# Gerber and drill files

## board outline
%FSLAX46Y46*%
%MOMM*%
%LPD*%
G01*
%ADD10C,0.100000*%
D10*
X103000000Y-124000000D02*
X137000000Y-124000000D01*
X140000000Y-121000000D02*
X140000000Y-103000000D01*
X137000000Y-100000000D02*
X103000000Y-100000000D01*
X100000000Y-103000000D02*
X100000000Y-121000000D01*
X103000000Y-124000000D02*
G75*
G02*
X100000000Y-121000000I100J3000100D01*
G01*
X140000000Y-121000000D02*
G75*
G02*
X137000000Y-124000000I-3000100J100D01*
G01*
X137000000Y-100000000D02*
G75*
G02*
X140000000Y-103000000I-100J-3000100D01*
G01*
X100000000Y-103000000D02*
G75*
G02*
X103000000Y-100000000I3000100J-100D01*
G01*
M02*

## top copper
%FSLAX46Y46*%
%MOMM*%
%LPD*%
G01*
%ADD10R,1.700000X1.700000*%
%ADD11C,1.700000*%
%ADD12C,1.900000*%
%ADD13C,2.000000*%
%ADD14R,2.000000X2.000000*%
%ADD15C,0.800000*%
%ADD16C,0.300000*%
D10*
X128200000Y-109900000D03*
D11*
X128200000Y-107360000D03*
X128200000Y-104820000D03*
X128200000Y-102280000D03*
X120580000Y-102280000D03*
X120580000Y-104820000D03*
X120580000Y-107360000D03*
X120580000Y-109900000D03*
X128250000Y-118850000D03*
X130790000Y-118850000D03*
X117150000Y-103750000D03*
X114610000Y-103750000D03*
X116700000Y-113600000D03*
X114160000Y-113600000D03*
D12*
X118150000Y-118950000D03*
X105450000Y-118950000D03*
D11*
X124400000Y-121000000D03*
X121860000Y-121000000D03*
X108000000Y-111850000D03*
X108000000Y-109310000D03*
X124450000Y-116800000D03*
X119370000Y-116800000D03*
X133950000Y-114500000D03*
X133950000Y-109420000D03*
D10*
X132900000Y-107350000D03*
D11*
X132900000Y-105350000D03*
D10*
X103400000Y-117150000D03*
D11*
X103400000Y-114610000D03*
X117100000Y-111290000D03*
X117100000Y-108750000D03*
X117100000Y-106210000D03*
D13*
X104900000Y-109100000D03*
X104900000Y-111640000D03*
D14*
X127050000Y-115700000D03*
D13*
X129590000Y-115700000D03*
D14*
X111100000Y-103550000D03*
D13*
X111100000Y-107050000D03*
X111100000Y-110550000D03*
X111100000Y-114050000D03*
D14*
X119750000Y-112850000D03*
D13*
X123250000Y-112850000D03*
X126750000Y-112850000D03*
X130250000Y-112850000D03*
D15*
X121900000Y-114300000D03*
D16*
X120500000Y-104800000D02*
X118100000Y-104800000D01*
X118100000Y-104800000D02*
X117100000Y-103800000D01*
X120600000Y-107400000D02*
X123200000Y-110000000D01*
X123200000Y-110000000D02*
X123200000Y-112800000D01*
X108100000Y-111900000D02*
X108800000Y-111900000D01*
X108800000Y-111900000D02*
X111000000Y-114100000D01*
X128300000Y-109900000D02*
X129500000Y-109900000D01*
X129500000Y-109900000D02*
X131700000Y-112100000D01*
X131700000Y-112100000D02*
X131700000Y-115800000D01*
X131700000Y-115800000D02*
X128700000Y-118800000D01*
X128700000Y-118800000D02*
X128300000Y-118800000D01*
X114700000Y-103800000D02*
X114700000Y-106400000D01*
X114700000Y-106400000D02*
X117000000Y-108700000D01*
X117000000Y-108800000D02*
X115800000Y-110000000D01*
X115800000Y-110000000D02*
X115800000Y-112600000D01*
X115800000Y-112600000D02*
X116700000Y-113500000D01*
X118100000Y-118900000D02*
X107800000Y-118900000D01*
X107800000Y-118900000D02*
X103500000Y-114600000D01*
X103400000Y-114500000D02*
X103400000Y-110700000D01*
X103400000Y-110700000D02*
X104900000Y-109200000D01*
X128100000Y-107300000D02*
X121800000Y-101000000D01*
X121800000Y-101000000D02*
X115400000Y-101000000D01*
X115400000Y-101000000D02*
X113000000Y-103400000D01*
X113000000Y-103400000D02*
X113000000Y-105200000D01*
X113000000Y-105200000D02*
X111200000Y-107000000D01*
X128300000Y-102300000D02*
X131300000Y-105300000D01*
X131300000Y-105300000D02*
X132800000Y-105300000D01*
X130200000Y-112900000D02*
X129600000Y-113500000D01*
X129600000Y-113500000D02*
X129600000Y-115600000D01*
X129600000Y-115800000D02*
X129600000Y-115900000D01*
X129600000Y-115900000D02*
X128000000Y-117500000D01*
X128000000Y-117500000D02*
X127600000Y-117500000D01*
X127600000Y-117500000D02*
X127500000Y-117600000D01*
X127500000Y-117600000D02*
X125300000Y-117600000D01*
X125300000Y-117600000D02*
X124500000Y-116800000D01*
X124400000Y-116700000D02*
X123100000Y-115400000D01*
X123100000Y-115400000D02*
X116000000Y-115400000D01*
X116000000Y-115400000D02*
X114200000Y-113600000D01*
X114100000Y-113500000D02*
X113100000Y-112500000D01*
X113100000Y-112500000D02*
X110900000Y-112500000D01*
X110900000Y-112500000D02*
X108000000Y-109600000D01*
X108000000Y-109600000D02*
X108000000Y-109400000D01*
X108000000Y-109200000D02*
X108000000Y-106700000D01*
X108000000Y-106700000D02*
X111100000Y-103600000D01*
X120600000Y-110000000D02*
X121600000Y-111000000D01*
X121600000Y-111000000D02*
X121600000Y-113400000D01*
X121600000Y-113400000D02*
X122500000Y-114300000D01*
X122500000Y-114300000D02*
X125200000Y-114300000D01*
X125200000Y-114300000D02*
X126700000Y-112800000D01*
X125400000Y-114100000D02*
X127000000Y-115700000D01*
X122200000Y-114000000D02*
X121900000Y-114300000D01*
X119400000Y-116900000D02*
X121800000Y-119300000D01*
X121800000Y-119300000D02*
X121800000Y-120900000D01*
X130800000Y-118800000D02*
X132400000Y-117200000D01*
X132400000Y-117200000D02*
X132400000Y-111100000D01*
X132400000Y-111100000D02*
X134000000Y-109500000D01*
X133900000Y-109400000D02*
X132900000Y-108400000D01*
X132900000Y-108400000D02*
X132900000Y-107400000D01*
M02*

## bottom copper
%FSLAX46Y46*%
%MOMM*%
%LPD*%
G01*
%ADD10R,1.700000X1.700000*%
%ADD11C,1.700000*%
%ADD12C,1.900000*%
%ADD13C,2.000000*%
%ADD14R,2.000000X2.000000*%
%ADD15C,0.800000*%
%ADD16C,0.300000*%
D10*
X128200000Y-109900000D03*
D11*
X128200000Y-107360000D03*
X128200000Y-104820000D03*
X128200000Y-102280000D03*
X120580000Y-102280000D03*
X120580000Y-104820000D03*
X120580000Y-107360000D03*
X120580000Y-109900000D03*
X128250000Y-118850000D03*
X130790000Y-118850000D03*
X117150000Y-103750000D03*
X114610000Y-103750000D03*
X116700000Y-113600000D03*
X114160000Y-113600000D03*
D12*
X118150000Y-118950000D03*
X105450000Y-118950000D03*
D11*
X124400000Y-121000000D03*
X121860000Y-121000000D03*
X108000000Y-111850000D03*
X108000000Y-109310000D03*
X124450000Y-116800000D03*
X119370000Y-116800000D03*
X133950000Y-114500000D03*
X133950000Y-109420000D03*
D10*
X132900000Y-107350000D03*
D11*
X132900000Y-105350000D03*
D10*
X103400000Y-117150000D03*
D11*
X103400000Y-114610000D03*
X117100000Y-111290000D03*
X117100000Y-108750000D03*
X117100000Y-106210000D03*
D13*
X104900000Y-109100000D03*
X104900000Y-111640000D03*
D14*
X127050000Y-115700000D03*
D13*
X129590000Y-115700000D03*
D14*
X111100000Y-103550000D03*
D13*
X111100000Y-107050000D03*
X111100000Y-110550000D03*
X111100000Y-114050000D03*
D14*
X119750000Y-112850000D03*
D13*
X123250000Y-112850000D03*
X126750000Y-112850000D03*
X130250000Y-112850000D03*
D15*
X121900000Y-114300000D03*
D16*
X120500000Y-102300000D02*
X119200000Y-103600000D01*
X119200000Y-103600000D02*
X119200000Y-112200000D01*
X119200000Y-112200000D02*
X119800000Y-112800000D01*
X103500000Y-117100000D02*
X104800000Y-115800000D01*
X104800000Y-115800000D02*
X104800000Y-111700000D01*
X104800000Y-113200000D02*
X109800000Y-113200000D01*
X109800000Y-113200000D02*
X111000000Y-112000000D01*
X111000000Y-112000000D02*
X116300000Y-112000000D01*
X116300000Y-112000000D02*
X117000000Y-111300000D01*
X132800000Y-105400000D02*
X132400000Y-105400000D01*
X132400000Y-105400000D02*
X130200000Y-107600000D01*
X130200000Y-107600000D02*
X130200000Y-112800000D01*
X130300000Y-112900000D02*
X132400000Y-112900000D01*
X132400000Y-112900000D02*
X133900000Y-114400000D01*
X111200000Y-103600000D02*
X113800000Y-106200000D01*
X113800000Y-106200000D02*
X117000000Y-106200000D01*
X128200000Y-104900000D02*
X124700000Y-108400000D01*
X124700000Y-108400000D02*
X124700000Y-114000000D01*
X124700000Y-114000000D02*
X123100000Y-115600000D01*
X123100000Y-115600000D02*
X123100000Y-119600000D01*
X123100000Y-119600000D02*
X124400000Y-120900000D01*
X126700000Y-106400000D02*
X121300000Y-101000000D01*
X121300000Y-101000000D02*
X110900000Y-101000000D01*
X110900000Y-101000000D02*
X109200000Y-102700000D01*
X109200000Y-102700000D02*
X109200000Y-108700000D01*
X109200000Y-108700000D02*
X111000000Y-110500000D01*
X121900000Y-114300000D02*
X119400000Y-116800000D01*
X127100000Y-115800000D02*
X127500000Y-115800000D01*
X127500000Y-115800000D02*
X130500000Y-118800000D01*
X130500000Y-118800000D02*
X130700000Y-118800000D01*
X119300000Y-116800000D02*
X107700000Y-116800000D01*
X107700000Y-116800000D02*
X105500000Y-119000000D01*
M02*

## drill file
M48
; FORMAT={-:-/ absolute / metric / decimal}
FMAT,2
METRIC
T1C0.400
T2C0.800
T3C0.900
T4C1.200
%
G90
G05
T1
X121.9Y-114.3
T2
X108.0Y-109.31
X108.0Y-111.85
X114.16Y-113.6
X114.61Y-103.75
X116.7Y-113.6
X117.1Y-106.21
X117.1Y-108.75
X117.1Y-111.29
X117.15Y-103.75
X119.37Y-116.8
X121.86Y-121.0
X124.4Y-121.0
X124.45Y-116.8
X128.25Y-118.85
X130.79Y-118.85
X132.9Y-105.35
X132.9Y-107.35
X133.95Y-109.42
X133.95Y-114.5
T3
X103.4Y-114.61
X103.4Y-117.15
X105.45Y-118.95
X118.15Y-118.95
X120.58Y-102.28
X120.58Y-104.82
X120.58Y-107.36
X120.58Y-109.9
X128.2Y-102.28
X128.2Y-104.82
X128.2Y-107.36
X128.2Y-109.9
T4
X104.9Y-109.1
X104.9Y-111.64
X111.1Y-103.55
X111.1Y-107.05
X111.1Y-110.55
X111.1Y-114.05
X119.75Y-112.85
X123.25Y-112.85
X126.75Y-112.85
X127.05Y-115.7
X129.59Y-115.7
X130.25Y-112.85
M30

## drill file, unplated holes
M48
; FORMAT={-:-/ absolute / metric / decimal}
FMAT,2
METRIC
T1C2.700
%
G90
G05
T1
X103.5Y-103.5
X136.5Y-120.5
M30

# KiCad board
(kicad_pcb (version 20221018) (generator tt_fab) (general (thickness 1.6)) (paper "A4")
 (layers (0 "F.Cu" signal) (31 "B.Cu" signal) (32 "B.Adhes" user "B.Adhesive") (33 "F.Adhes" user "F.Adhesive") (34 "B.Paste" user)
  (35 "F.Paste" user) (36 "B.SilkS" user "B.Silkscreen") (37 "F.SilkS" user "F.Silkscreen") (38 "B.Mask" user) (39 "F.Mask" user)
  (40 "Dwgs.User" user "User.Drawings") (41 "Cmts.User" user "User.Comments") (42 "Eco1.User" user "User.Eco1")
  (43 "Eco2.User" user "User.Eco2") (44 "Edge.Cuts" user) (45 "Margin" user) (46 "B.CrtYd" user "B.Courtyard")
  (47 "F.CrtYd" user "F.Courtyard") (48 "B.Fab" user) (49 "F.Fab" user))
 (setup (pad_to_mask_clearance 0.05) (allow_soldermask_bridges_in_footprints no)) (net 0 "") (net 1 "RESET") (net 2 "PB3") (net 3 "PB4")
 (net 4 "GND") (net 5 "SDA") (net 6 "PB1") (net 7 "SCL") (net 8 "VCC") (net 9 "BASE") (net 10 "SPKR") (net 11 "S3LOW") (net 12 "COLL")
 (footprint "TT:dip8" (layer "F.Cu") (at 128.2 109.9)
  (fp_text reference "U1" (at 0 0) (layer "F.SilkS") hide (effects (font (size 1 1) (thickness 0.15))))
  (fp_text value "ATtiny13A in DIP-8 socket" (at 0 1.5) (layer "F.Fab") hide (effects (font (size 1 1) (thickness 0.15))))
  (pad "1" thru_hole rect (at 0 0) (size 1.7 1.7) (drill 0.9) (layers "*.Cu" "*.Mask") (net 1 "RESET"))
  (pad "2" thru_hole circle (at 0 -2.54) (size 1.7 1.7) (drill 0.9) (layers "*.Cu" "*.Mask") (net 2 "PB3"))
  (pad "3" thru_hole circle (at 0 -5.08) (size 1.7 1.7) (drill 0.9) (layers "*.Cu" "*.Mask") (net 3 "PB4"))
  (pad "4" thru_hole circle (at 0 -7.62) (size 1.7 1.7) (drill 0.9) (layers "*.Cu" "*.Mask") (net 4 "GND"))
  (pad "5" thru_hole circle (at -7.62 -7.62) (size 1.7 1.7) (drill 0.9) (layers "*.Cu" "*.Mask") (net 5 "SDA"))
  (pad "6" thru_hole circle (at -7.62 -5.08) (size 1.7 1.7) (drill 0.9) (layers "*.Cu" "*.Mask") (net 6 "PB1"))
  (pad "7" thru_hole circle (at -7.62 -2.54) (size 1.7 1.7) (drill 0.9) (layers "*.Cu" "*.Mask") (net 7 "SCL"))
  (pad "8" thru_hole circle (at -7.62 0) (size 1.7 1.7) (drill 0.9) (layers "*.Cu" "*.Mask") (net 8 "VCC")))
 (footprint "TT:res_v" (layer "F.Cu") (at 128.25 118.85)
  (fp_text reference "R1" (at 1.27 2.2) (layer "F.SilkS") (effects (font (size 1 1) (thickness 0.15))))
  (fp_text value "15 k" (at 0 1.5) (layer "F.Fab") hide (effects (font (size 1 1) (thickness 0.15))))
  (pad "1" thru_hole circle (at 0 0) (size 1.7 1.7) (drill 0.8) (layers "*.Cu" "*.Mask") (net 1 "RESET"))
  (pad "2" thru_hole circle (at 2.54 0) (size 1.7 1.7) (drill 0.8) (layers "*.Cu" "*.Mask") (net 8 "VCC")))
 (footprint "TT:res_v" (layer "F.Cu") (at 117.15 103.75)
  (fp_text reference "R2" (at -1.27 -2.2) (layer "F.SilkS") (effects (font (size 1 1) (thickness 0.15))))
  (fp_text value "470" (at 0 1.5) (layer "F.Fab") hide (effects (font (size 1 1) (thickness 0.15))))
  (pad "1" thru_hole circle (at 0 0) (size 1.7 1.7) (drill 0.8) (layers "*.Cu" "*.Mask") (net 6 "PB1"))
  (pad "2" thru_hole circle (at -2.54 0) (size 1.7 1.7) (drill 0.8) (layers "*.Cu" "*.Mask") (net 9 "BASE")))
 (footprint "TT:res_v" (layer "F.Cu") (at 116.7 113.6)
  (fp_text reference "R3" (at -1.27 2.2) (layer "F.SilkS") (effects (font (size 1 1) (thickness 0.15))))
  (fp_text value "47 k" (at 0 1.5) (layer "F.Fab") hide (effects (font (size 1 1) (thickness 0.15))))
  (pad "1" thru_hole circle (at 0 0) (size 1.7 1.7) (drill 0.8) (layers "*.Cu" "*.Mask") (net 9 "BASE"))
  (pad "2" thru_hole circle (at -2.54 0) (size 1.7 1.7) (drill 0.8) (layers "*.Cu" "*.Mask") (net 4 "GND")))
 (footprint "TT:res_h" (layer "F.Cu") (at 118.15 118.95)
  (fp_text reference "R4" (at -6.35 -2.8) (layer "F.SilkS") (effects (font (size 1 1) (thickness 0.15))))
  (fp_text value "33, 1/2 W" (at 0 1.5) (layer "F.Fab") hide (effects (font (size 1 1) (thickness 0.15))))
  (pad "1" thru_hole circle (at 0 0) (size 1.9 1.9) (drill 0.9) (layers "*.Cu" "*.Mask") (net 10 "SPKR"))
  (pad "2" thru_hole circle (at -12.7 0) (size 1.9 1.9) (drill 0.9) (layers "*.Cu" "*.Mask") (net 8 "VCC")))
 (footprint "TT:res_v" (layer "F.Cu") (at 124.4 121)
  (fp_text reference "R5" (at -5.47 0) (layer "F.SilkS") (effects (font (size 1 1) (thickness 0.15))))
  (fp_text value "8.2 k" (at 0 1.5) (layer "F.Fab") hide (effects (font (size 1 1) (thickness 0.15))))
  (pad "1" thru_hole circle (at 0 0) (size 1.7 1.7) (drill 0.8) (layers "*.Cu" "*.Mask") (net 3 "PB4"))
  (pad "2" thru_hole circle (at -2.54 0) (size 1.7 1.7) (drill 0.8) (layers "*.Cu" "*.Mask") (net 8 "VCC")))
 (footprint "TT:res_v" (layer "F.Cu") (at 108 111.85)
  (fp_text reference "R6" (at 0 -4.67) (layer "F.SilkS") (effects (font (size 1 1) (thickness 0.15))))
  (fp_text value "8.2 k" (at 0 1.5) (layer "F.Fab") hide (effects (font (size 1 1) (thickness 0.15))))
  (pad "1" thru_hole circle (at 0 0) (size 1.7 1.7) (drill 0.8) (layers "*.Cu" "*.Mask") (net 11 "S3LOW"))
  (pad "2" thru_hole circle (at 0 -2.54) (size 1.7 1.7) (drill 0.8) (layers "*.Cu" "*.Mask") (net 4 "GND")))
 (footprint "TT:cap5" (layer "F.Cu") (at 124.45 116.8)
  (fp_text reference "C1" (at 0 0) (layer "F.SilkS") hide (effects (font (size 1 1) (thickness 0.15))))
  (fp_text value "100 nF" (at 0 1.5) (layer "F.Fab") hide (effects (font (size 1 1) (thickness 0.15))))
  (pad "1" thru_hole circle (at 0 0) (size 1.7 1.7) (drill 0.8) (layers "*.Cu" "*.Mask") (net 4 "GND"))
  (pad "2" thru_hole circle (at -5.08 0) (size 1.7 1.7) (drill 0.8) (layers "*.Cu" "*.Mask") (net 8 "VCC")))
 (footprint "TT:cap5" (layer "F.Cu") (at 133.95 114.5)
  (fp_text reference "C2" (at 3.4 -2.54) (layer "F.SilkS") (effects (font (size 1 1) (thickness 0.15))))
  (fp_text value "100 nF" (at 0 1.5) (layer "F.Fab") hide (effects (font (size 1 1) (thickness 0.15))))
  (pad "1" thru_hole circle (at 0 0) (size 1.7 1.7) (drill 0.8) (layers "*.Cu" "*.Mask") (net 4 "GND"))
  (pad "2" thru_hole circle (at 0 -5.08) (size 1.7 1.7) (drill 0.8) (layers "*.Cu" "*.Mask") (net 8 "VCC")))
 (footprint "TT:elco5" (layer "F.Cu") (at 132.9 107.35)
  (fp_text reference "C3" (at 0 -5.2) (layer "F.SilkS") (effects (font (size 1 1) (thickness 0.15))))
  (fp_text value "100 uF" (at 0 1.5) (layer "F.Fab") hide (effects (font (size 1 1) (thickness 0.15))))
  (pad "+" thru_hole rect (at 0 0) (size 1.7 1.7) (drill 0.8) (layers "*.Cu" "*.Mask") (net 8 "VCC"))
  (pad "-" thru_hole circle (at 0 -2) (size 1.7 1.7) (drill 0.8) (layers "*.Cu" "*.Mask") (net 4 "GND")))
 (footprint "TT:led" (layer "F.Cu") (at 103.4 117.15)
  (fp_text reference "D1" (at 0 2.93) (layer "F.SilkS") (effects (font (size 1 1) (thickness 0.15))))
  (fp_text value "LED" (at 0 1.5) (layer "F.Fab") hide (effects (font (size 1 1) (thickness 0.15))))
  (pad "A" thru_hole rect (at 0 0) (size 1.7 1.7) (drill 0.9) (layers "*.Cu" "*.Mask") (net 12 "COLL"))
  (pad "K" thru_hole circle (at 0 -2.54) (size 1.7 1.7) (drill 0.9) (layers "*.Cu" "*.Mask") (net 10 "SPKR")))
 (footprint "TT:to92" (layer "F.Cu") (at 117.1 108.75)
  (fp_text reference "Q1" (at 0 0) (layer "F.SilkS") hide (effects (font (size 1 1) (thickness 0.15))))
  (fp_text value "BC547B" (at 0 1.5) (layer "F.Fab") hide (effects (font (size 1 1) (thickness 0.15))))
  (pad "C" thru_hole circle (at 0 2.54) (size 1.7 1.7) (drill 0.8) (layers "*.Cu" "*.Mask") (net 12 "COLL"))
  (pad "B" thru_hole circle (at 0 0) (size 1.7 1.7) (drill 0.8) (layers "*.Cu" "*.Mask") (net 9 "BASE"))
  (pad "E" thru_hole circle (at 0 -2.54) (size 1.7 1.7) (drill 0.8) (layers "*.Cu" "*.Mask") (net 4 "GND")))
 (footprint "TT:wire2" (layer "F.Cu") (at 104.9 109.1)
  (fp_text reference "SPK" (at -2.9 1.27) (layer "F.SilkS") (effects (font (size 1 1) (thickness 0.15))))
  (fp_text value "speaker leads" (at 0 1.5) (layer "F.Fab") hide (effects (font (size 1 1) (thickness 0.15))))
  (pad "1" thru_hole circle (at 0 0) (size 2 2) (drill 1.2) (layers "*.Cu" "*.Mask") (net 10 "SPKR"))
  (pad "2" thru_hole circle (at 0 2.54) (size 2 2) (drill 1.2) (layers "*.Cu" "*.Mask") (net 12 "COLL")))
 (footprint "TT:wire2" (layer "F.Cu") (at 127.05 115.7)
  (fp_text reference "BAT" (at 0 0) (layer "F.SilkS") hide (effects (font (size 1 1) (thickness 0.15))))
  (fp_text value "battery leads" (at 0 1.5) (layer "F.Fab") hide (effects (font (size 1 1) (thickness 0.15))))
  (pad "1" thru_hole rect (at 0 0) (size 2 2) (drill 1.2) (layers "*.Cu" "*.Mask") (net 8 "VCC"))
  (pad "2" thru_hole circle (at 2.54 0) (size 2 2) (drill 1.2) (layers "*.Cu" "*.Mask") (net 4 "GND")))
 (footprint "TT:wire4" (layer "F.Cu") (at 111.1 103.55)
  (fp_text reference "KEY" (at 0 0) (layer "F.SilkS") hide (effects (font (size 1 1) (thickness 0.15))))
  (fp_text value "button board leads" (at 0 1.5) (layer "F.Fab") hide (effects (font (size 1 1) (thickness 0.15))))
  (pad "1" thru_hole rect (at 0 0) (size 2 2) (drill 1.2) (layers "*.Cu" "*.Mask") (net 4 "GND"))
  (pad "2" thru_hole circle (at 0 3.5) (size 2 2) (drill 1.2) (layers "*.Cu" "*.Mask") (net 2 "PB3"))
  (pad "3" thru_hole circle (at 0 7) (size 2 2) (drill 1.2) (layers "*.Cu" "*.Mask") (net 3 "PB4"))
  (pad "4" thru_hole circle (at 0 10.5) (size 2 2) (drill 1.2) (layers "*.Cu" "*.Mask") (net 11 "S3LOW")))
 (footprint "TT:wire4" (layer "F.Cu") (at 119.75 112.85)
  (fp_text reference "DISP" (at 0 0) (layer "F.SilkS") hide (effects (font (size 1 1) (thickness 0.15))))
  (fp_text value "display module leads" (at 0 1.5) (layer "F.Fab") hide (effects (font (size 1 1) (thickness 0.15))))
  (pad "1" thru_hole rect (at 0 0) (size 2 2) (drill 1.2) (layers "*.Cu" "*.Mask") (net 5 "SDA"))
  (pad "2" thru_hole circle (at 3.5 0) (size 2 2) (drill 1.2) (layers "*.Cu" "*.Mask") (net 7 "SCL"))
  (pad "3" thru_hole circle (at 7 0) (size 2 2) (drill 1.2) (layers "*.Cu" "*.Mask") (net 8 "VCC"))
  (pad "4" thru_hole circle (at 10.5 0) (size 2 2) (drill 1.2) (layers "*.Cu" "*.Mask") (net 4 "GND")))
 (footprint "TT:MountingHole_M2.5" (layer "F.Cu") (at 136.5 120.5)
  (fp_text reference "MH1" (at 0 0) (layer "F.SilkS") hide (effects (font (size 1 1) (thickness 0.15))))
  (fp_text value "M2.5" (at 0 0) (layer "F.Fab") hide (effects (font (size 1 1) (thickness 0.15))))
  (pad "" np_thru_hole circle (at 0 0) (size 2.7 2.7) (drill 2.7) (layers "*.Cu" "*.Mask")))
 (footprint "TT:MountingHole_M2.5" (layer "F.Cu") (at 103.5 103.5)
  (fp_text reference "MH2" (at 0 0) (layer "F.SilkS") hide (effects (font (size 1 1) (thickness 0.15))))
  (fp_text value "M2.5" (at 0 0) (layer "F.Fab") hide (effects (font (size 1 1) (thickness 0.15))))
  (pad "" np_thru_hole circle (at 0 0) (size 2.7 2.7) (drill 2.7) (layers "*.Cu" "*.Mask")))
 (gr_line (start 103 124) (end 137 124) (stroke (width 0.1) (type solid)) (layer "Edge.Cuts"))
 (gr_line (start 140 121) (end 140 103) (stroke (width 0.1) (type solid)) (layer "Edge.Cuts"))
 (gr_line (start 137 100) (end 103 100) (stroke (width 0.1) (type solid)) (layer "Edge.Cuts"))
 (gr_line (start 100 103) (end 100 121) (stroke (width 0.1) (type solid)) (layer "Edge.Cuts"))
 (gr_arc (start 100 121) (mid 100.8787 123.1213) (end 103 124) (stroke (width 0.1) (type solid)) (layer "Edge.Cuts"))
 (gr_arc (start 137 124) (mid 139.1213 123.1213) (end 140 121) (stroke (width 0.1) (type solid)) (layer "Edge.Cuts"))
 (gr_arc (start 140 103) (mid 139.1213 100.8787) (end 137 100) (stroke (width 0.1) (type solid)) (layer "Edge.Cuts"))
 (gr_arc (start 103 100) (mid 100.8787 100.8787) (end 100 103) (stroke (width 0.1) (type solid)) (layer "Edge.Cuts"))
 (segment (start 120.5 104.8) (end 118.1 104.8) (width 0.3) (layer "F.Cu") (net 6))
 (segment (start 118.1 104.8) (end 117.1 103.8) (width 0.3) (layer "F.Cu") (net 6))
 (segment (start 120.6 107.4) (end 123.2 110) (width 0.3) (layer "F.Cu") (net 7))
 (segment (start 123.2 110) (end 123.2 112.8) (width 0.3) (layer "F.Cu") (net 7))
 (segment (start 108.1 111.9) (end 108.8 111.9) (width 0.3) (layer "F.Cu") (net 11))
 (segment (start 108.8 111.9) (end 111 114.1) (width 0.3) (layer "F.Cu") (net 11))
 (segment (start 120.5 102.3) (end 119.2 103.6) (width 0.3) (layer "B.Cu") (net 5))
 (segment (start 119.2 103.6) (end 119.2 112.2) (width 0.3) (layer "B.Cu") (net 5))
 (segment (start 119.2 112.2) (end 119.8 112.8) (width 0.3) (layer "B.Cu") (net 5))
 (segment (start 128.3 109.9) (end 129.5 109.9) (width 0.3) (layer "F.Cu") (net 1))
 (segment (start 129.5 109.9) (end 131.7 112.1) (width 0.3) (layer "F.Cu") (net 1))
 (segment (start 131.7 112.1) (end 131.7 115.8) (width 0.3) (layer "F.Cu") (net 1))
 (segment (start 131.7 115.8) (end 128.7 118.8) (width 0.3) (layer "F.Cu") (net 1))
 (segment (start 128.7 118.8) (end 128.3 118.8) (width 0.3) (layer "F.Cu") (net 1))
 (segment (start 114.7 103.8) (end 114.7 106.4) (width 0.3) (layer "F.Cu") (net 9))
 (segment (start 114.7 106.4) (end 117 108.7) (width 0.3) (layer "F.Cu") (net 9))
 (segment (start 117 108.8) (end 115.8 110) (width 0.3) (layer "F.Cu") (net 9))
 (segment (start 115.8 110) (end 115.8 112.6) (width 0.3) (layer "F.Cu") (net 9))
 (segment (start 115.8 112.6) (end 116.7 113.5) (width 0.3) (layer "F.Cu") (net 9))
 (segment (start 118.1 118.9) (end 107.8 118.9) (width 0.3) (layer "F.Cu") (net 10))
 (segment (start 107.8 118.9) (end 103.5 114.6) (width 0.3) (layer "F.Cu") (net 10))
 (segment (start 103.4 114.5) (end 103.4 110.7) (width 0.3) (layer "F.Cu") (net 10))
 (segment (start 103.4 110.7) (end 104.9 109.2) (width 0.3) (layer "F.Cu") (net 10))
 (segment (start 128.1 107.3) (end 121.8 101) (width 0.3) (layer "F.Cu") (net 2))
 (segment (start 121.8 101) (end 115.4 101) (width 0.3) (layer "F.Cu") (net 2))
 (segment (start 115.4 101) (end 113 103.4) (width 0.3) (layer "F.Cu") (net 2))
 (segment (start 113 103.4) (end 113 105.2) (width 0.3) (layer "F.Cu") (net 2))
 (segment (start 113 105.2) (end 111.2 107) (width 0.3) (layer "F.Cu") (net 2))
 (segment (start 103.5 117.1) (end 104.8 115.8) (width 0.3) (layer "B.Cu") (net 12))
 (segment (start 104.8 115.8) (end 104.8 111.7) (width 0.3) (layer "B.Cu") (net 12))
 (segment (start 104.8 113.2) (end 109.8 113.2) (width 0.3) (layer "B.Cu") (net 12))
 (segment (start 109.8 113.2) (end 111 112) (width 0.3) (layer "B.Cu") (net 12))
 (segment (start 111 112) (end 116.3 112) (width 0.3) (layer "B.Cu") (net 12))
 (segment (start 116.3 112) (end 117 111.3) (width 0.3) (layer "B.Cu") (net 12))
 (segment (start 128.3 102.3) (end 131.3 105.3) (width 0.3) (layer "F.Cu") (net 4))
 (segment (start 131.3 105.3) (end 132.8 105.3) (width 0.3) (layer "F.Cu") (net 4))
 (segment (start 130.2 112.9) (end 129.6 113.5) (width 0.3) (layer "F.Cu") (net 4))
 (segment (start 129.6 113.5) (end 129.6 115.6) (width 0.3) (layer "F.Cu") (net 4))
 (segment (start 129.6 115.8) (end 129.6 115.9) (width 0.3) (layer "F.Cu") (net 4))
 (segment (start 129.6 115.9) (end 128 117.5) (width 0.3) (layer "F.Cu") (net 4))
 (segment (start 128 117.5) (end 127.6 117.5) (width 0.3) (layer "F.Cu") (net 4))
 (segment (start 127.6 117.5) (end 127.5 117.6) (width 0.3) (layer "F.Cu") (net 4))
 (segment (start 127.5 117.6) (end 125.3 117.6) (width 0.3) (layer "F.Cu") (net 4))
 (segment (start 125.3 117.6) (end 124.5 116.8) (width 0.3) (layer "F.Cu") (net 4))
 (segment (start 124.4 116.7) (end 123.1 115.4) (width 0.3) (layer "F.Cu") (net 4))
 (segment (start 123.1 115.4) (end 116 115.4) (width 0.3) (layer "F.Cu") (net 4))
 (segment (start 116 115.4) (end 114.2 113.6) (width 0.3) (layer "F.Cu") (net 4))
 (segment (start 114.1 113.5) (end 113.1 112.5) (width 0.3) (layer "F.Cu") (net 4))
 (segment (start 113.1 112.5) (end 110.9 112.5) (width 0.3) (layer "F.Cu") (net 4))
 (segment (start 110.9 112.5) (end 108 109.6) (width 0.3) (layer "F.Cu") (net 4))
 (segment (start 108 109.6) (end 108 109.4) (width 0.3) (layer "F.Cu") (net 4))
 (segment (start 108 109.2) (end 108 106.7) (width 0.3) (layer "F.Cu") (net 4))
 (segment (start 108 106.7) (end 111.1 103.6) (width 0.3) (layer "F.Cu") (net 4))
 (segment (start 132.8 105.4) (end 132.4 105.4) (width 0.3) (layer "B.Cu") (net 4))
 (segment (start 132.4 105.4) (end 130.2 107.6) (width 0.3) (layer "B.Cu") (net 4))
 (segment (start 130.2 107.6) (end 130.2 112.8) (width 0.3) (layer "B.Cu") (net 4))
 (segment (start 130.3 112.9) (end 132.4 112.9) (width 0.3) (layer "B.Cu") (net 4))
 (segment (start 132.4 112.9) (end 133.9 114.4) (width 0.3) (layer "B.Cu") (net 4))
 (segment (start 111.2 103.6) (end 113.8 106.2) (width 0.3) (layer "B.Cu") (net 4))
 (segment (start 113.8 106.2) (end 117 106.2) (width 0.3) (layer "B.Cu") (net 4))
 (segment (start 128.2 104.9) (end 124.7 108.4) (width 0.3) (layer "B.Cu") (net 3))
 (segment (start 124.7 108.4) (end 124.7 114) (width 0.3) (layer "B.Cu") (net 3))
 (segment (start 124.7 114) (end 123.1 115.6) (width 0.3) (layer "B.Cu") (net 3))
 (segment (start 123.1 115.6) (end 123.1 119.6) (width 0.3) (layer "B.Cu") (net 3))
 (segment (start 123.1 119.6) (end 124.4 120.9) (width 0.3) (layer "B.Cu") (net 3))
 (segment (start 126.7 106.4) (end 121.3 101) (width 0.3) (layer "B.Cu") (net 3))
 (segment (start 121.3 101) (end 110.9 101) (width 0.3) (layer "B.Cu") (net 3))
 (segment (start 110.9 101) (end 109.2 102.7) (width 0.3) (layer "B.Cu") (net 3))
 (segment (start 109.2 102.7) (end 109.2 108.7) (width 0.3) (layer "B.Cu") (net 3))
 (segment (start 109.2 108.7) (end 111 110.5) (width 0.3) (layer "B.Cu") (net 3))
 (segment (start 120.6 110) (end 121.6 111) (width 0.3) (layer "F.Cu") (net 8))
 (segment (start 121.6 111) (end 121.6 113.4) (width 0.3) (layer "F.Cu") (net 8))
 (segment (start 121.6 113.4) (end 122.5 114.3) (width 0.3) (layer "F.Cu") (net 8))
 (segment (start 122.5 114.3) (end 125.2 114.3) (width 0.3) (layer "F.Cu") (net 8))
 (segment (start 125.2 114.3) (end 126.7 112.8) (width 0.3) (layer "F.Cu") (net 8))
 (segment (start 125.4 114.1) (end 127 115.7) (width 0.3) (layer "F.Cu") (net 8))
 (segment (start 122.2 114) (end 121.9 114.3) (width 0.3) (layer "F.Cu") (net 8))
 (segment (start 119.4 116.9) (end 121.8 119.3) (width 0.3) (layer "F.Cu") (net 8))
 (segment (start 121.8 119.3) (end 121.8 120.9) (width 0.3) (layer "F.Cu") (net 8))
 (segment (start 130.8 118.8) (end 132.4 117.2) (width 0.3) (layer "F.Cu") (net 8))
 (segment (start 132.4 117.2) (end 132.4 111.1) (width 0.3) (layer "F.Cu") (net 8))
 (segment (start 132.4 111.1) (end 134 109.5) (width 0.3) (layer "F.Cu") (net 8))
 (segment (start 133.9 109.4) (end 132.9 108.4) (width 0.3) (layer "F.Cu") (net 8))
 (segment (start 132.9 108.4) (end 132.9 107.4) (width 0.3) (layer "F.Cu") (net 8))
 (segment (start 121.9 114.3) (end 119.4 116.8) (width 0.3) (layer "B.Cu") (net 8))
 (segment (start 127.1 115.8) (end 127.5 115.8) (width 0.3) (layer "B.Cu") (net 8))
 (segment (start 127.5 115.8) (end 130.5 118.8) (width 0.3) (layer "B.Cu") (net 8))
 (segment (start 130.5 118.8) (end 130.7 118.8) (width 0.3) (layer "B.Cu") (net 8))
 (segment (start 119.3 116.8) (end 107.7 116.8) (width 0.3) (layer "B.Cu") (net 8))
 (segment (start 107.7 116.8) (end 105.5 119) (width 0.3) (layer "B.Cu") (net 8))
 (via (at 121.9 114.3) (size 0.8) (drill 0.4) (layers "F.Cu" "B.Cu") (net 8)))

